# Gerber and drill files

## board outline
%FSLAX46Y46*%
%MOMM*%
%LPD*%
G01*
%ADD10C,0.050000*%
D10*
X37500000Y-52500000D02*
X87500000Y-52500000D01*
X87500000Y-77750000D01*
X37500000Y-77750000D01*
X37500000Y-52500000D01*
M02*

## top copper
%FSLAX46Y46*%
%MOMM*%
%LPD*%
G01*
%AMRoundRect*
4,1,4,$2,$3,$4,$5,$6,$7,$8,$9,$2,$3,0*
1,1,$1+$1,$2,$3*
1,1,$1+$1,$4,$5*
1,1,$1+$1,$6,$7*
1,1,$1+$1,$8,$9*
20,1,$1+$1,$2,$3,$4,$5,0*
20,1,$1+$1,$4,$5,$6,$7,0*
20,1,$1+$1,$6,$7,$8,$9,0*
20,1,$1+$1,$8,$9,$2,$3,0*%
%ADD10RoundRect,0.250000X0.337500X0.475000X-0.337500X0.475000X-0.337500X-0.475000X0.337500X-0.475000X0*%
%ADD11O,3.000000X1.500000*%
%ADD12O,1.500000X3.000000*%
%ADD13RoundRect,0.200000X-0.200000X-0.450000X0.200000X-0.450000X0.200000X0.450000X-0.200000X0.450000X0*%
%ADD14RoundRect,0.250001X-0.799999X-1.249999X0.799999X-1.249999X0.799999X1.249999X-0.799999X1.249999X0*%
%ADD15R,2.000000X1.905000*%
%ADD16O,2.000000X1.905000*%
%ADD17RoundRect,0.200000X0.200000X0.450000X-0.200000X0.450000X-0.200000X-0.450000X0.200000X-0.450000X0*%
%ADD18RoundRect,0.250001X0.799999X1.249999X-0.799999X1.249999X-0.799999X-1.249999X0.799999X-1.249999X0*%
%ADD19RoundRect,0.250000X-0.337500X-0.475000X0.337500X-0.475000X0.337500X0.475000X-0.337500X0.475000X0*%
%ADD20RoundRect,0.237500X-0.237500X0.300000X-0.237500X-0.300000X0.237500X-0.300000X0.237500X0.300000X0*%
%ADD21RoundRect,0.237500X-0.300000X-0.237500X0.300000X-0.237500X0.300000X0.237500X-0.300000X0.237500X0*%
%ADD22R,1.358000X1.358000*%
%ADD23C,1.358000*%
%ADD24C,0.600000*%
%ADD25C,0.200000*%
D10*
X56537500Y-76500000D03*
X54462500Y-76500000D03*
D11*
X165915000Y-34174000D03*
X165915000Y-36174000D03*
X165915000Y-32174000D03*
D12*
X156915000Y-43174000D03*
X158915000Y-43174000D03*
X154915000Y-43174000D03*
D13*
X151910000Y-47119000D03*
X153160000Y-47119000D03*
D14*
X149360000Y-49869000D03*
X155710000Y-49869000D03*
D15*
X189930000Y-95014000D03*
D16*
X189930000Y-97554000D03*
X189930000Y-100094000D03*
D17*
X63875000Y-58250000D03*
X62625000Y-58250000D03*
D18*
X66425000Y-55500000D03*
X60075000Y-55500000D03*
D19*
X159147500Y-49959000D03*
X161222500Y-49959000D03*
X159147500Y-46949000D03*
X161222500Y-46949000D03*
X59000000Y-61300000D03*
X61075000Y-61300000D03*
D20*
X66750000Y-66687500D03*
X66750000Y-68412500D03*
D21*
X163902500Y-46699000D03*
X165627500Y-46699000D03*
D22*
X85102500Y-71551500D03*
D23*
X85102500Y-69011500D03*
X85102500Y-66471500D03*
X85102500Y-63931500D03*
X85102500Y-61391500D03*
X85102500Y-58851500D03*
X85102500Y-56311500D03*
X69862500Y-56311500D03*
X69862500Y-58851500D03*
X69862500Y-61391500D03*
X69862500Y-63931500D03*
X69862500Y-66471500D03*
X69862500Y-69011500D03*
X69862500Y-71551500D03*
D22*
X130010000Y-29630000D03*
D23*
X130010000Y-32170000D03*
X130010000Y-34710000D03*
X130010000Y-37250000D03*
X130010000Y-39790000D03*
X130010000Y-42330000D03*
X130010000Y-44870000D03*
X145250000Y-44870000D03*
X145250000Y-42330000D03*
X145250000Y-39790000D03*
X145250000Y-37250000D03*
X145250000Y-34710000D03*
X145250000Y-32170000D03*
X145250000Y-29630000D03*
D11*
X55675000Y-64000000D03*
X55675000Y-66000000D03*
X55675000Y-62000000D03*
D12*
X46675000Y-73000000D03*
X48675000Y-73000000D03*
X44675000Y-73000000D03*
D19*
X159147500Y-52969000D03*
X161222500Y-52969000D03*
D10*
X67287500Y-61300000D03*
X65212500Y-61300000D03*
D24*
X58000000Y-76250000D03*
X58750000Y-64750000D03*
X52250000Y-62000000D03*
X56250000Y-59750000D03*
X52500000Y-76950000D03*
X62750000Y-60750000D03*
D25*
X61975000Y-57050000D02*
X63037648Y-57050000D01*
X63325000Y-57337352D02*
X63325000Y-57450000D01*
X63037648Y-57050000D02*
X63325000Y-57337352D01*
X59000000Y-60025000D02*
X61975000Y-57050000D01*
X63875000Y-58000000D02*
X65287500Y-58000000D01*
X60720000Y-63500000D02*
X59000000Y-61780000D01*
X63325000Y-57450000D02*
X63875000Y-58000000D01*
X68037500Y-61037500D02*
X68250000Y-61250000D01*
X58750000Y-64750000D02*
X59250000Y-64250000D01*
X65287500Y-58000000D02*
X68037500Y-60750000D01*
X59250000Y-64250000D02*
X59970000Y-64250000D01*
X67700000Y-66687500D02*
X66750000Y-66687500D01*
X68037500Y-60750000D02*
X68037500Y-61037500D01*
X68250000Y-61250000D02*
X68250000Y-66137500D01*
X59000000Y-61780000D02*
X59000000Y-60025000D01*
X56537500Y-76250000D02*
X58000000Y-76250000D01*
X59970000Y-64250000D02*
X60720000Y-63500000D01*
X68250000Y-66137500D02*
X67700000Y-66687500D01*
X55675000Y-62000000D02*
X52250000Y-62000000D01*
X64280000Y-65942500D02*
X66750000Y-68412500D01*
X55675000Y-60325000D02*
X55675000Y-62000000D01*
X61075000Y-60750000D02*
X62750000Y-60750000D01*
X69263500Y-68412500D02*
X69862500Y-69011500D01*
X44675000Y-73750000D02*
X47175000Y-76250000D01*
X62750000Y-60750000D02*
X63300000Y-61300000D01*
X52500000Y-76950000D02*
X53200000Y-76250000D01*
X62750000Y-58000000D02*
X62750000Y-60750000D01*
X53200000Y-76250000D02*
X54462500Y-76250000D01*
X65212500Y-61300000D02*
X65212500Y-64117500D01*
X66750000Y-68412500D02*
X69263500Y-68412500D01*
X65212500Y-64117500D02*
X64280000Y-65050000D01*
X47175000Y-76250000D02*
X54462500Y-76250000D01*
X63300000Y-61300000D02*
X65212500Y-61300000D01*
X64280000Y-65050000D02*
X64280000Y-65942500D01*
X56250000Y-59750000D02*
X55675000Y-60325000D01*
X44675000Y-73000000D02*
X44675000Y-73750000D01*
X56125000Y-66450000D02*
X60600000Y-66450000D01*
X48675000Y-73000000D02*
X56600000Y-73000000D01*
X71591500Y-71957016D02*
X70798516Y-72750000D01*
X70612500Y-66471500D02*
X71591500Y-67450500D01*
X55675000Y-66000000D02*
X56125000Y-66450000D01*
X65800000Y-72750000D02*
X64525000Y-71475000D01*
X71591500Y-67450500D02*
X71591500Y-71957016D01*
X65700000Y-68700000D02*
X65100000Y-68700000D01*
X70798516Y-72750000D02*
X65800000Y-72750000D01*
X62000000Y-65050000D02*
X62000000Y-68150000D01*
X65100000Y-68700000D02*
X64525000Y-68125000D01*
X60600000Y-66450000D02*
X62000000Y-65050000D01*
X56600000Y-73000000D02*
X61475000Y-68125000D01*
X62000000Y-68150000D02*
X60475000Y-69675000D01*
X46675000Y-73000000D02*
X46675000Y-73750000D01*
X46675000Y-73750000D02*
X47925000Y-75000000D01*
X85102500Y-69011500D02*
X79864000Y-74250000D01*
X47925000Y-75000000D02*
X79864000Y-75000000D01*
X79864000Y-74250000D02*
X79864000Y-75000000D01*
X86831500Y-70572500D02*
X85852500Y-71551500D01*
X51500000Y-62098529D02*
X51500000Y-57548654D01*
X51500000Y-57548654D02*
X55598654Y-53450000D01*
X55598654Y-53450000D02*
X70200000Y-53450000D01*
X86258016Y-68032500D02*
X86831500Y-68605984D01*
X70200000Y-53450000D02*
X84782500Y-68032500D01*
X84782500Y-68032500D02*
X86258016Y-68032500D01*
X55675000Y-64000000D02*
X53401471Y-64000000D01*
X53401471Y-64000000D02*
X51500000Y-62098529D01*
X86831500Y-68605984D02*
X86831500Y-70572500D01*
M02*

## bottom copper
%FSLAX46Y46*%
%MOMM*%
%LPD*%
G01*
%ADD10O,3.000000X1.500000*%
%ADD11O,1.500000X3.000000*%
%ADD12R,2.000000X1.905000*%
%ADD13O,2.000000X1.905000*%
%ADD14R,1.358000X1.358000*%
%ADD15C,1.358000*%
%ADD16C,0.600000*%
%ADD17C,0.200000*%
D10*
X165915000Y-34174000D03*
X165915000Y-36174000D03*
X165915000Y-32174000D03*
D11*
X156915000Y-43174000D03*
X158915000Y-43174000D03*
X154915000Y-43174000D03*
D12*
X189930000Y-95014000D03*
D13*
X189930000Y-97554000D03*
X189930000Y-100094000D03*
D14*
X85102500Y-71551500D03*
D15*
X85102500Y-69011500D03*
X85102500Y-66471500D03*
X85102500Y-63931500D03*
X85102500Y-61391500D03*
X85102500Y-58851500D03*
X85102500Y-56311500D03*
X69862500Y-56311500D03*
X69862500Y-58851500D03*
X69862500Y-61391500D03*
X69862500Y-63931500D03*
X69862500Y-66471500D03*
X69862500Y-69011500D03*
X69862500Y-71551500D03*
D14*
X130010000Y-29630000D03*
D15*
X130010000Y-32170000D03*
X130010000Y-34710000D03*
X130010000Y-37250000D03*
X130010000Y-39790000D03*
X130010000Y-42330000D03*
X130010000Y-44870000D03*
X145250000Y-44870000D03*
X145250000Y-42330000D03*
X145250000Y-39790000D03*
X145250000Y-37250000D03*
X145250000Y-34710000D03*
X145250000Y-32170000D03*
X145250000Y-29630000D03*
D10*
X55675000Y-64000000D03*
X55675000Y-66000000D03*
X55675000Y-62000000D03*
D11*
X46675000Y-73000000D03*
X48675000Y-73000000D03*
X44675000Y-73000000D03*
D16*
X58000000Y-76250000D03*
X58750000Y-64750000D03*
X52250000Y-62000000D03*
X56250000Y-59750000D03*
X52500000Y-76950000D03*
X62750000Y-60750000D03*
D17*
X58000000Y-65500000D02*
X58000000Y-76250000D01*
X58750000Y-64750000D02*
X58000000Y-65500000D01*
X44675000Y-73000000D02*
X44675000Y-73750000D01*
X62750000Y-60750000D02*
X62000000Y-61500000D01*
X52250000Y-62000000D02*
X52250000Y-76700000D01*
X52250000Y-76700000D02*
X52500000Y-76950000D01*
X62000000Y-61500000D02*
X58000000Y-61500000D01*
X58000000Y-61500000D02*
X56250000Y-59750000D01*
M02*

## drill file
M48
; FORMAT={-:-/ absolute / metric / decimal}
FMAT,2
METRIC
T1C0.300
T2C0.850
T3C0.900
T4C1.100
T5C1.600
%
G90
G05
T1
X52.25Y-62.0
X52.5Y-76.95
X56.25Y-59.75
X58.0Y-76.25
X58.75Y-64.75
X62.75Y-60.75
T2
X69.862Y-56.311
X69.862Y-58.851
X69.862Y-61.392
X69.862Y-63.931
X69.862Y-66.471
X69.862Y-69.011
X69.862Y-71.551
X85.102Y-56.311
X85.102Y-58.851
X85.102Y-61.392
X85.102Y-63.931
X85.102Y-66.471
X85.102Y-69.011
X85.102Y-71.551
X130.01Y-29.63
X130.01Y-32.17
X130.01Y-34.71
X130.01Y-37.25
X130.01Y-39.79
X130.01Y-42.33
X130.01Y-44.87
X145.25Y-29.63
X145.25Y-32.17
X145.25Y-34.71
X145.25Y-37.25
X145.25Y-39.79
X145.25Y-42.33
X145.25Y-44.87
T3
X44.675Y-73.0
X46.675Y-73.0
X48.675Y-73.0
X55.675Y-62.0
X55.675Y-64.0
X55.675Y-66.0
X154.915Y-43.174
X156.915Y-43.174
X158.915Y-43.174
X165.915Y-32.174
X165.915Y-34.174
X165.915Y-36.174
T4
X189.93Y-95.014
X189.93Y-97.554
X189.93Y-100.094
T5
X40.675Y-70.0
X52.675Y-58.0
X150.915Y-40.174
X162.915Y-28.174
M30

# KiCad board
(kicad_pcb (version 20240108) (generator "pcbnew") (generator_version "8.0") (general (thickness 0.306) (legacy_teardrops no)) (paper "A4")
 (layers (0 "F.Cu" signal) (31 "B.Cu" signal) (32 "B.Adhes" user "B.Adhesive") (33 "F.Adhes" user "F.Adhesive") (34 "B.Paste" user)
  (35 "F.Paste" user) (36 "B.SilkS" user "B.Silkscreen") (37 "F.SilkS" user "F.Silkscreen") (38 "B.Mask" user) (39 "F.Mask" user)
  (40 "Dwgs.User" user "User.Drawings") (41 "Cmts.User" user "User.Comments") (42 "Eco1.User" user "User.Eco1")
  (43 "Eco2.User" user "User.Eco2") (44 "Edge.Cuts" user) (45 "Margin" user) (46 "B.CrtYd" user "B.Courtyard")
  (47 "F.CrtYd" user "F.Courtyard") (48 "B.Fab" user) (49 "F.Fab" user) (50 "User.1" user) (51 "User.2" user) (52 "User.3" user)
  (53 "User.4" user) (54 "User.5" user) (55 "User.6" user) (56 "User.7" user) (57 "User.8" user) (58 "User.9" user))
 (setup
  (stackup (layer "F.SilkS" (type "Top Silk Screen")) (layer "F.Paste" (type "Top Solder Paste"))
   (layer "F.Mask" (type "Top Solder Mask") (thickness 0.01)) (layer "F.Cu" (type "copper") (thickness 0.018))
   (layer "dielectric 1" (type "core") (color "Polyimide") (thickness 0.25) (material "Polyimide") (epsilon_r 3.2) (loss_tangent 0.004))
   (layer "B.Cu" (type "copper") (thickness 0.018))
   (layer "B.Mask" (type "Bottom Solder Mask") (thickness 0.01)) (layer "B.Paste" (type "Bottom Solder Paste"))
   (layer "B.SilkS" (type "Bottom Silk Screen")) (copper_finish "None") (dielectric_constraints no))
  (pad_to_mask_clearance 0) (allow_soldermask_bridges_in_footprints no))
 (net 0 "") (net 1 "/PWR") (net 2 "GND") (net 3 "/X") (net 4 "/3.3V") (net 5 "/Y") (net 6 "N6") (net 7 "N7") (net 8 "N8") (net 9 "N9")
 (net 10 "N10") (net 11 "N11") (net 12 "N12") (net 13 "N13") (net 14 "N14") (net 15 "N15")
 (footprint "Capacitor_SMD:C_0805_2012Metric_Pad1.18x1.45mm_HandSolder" (layer "F.Cu") (at 55.5 76.5 180)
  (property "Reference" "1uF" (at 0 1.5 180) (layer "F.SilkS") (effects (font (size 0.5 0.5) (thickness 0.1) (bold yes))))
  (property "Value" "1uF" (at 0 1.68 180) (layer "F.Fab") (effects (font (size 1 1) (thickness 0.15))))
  (pad "1" smd roundrect (at -1.0375 0 180) (size 1.175 1.45) (layers "F.Cu" "F.Paste" "F.Mask") (roundrect_rratio 0.212766) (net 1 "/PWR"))
  (pad "2" smd roundrect (at 1.0375 0 180) (size 1.175 1.45) (layers "F.Cu" "F.Paste" "F.Mask") (roundrect_rratio 0.212766) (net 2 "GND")))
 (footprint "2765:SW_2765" (layer "F.Cu") (at 156.915 34.174)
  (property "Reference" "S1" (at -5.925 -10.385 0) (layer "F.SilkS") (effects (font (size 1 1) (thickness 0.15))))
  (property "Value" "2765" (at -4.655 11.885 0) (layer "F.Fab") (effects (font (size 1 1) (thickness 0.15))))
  (pad "" np_thru_hole circle (at -6 6) (size 1.6 1.6) (drill 1.6) (layers "*.Cu" "*.Mask"))
  (pad "" np_thru_hole circle (at 6 -6) (size 1.6 1.6) (drill 1.6) (layers "*.Cu" "*.Mask"))
  (pad "X" thru_hole oval (at 9 0) (size 3 1.5) (drill 0.9) (layers "*.Cu" "*.Mask") (remove_unused_layers no) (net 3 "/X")
   (solder_mask_margin 0.102))
  (pad "X+" thru_hole oval (at 9 2) (size 3 1.5) (drill 0.9) (layers "*.Cu" "*.Mask") (remove_unused_layers no) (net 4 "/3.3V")
   (solder_mask_margin 0.102))
  (pad "X-" thru_hole oval (at 9 -2) (size 3 1.5) (drill 0.9) (layers "*.Cu" "*.Mask") (remove_unused_layers no) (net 2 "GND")
   (solder_mask_margin 0.102))
  (pad "Y" thru_hole oval (at 0 9) (size 1.5 3) (drill 0.9) (layers "*.Cu" "*.Mask") (remove_unused_layers no) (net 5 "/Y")
   (solder_mask_margin 0.102))
  (pad "Y+" thru_hole oval (at 2 9) (size 1.5 3) (drill 0.9) (layers "*.Cu" "*.Mask") (remove_unused_layers no) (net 4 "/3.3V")
   (solder_mask_margin 0.102))
  (pad "Y-" thru_hole oval (at -2 9) (size 1.5 3) (drill 0.9) (layers "*.Cu" "*.Mask") (remove_unused_layers no) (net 2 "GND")
   (solder_mask_margin 0.102)))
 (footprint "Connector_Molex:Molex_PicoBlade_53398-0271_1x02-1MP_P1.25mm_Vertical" (layer "F.Cu") (at 152.535 48.369)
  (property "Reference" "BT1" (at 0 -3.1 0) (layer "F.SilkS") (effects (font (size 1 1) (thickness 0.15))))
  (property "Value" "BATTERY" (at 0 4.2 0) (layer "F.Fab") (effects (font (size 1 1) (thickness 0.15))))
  (pad "1" smd roundrect (at -0.625 -1.25) (size 0.8 1.3) (layers "F.Cu" "F.Paste" "F.Mask") (roundrect_rratio 0.25) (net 1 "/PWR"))
  (pad "2" smd roundrect (at 0.625 -1.25) (size 0.8 1.3) (layers "F.Cu" "F.Paste" "F.Mask") (roundrect_rratio 0.25) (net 2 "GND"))
  (pad "MP" smd roundrect (at -3.175 1.5) (size 2.1 3) (layers "F.Cu" "F.Paste" "F.Mask") (roundrect_rratio 0.119048))
  (pad "MP" smd roundrect (at 3.175 1.5) (size 2.1 3) (layers "F.Cu" "F.Paste" "F.Mask") (roundrect_rratio 0.119048)))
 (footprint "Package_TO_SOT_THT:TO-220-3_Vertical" (layer "F.Cu") (at 189.93 95.014 -90)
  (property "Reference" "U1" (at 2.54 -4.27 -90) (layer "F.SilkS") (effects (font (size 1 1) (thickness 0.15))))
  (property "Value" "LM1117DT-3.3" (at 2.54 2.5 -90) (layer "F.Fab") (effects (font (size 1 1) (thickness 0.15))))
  (pad "1" thru_hole rect (at 0 0 270) (size 1.905 2) (drill 1.1) (layers "*.Cu" "*.Mask") (remove_unused_layers no) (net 2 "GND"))
  (pad "2" thru_hole oval (at 2.54 0 270) (size 1.905 2) (drill 1.1) (layers "*.Cu" "*.Mask") (remove_unused_layers no) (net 4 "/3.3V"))
  (pad "3" thru_hole oval (at 5.08 0 270) (size 1.905 2) (drill 1.1) (layers "*.Cu" "*.Mask") (remove_unused_layers no) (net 1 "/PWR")))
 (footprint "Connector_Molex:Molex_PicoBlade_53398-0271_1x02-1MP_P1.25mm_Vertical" (layer "F.Cu") (at 63.25 57 180)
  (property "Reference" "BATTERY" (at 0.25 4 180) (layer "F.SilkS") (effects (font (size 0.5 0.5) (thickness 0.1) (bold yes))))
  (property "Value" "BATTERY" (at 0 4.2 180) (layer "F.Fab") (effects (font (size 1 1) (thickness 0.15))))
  (pad "1" smd roundrect (at -0.625 -1.25 180) (size 0.8 1.3) (layers "F.Cu" "F.Paste" "F.Mask") (roundrect_rratio 0.25) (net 1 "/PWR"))
  (pad "2" smd roundrect (at 0.625 -1.25 180) (size 0.8 1.3) (layers "F.Cu" "F.Paste" "F.Mask") (roundrect_rratio 0.25) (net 2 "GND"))
  (pad "MP" smd roundrect (at -3.175 1.5 180) (size 2.1 3) (layers "F.Cu" "F.Paste" "F.Mask") (roundrect_rratio 0.119048))
  (pad "MP" smd roundrect (at 3.175 1.5 180) (size 2.1 3) (layers "F.Cu" "F.Paste" "F.Mask") (roundrect_rratio 0.119048)))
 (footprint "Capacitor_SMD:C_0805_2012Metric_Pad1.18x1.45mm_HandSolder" (layer "F.Cu") (at 160.185 49.959)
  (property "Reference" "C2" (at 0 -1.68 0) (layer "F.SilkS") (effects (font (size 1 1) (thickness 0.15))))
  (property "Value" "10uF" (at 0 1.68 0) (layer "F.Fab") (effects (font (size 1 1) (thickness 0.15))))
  (pad "1" smd roundrect (at -1.0375 0) (size 1.175 1.45) (layers "F.Cu" "F.Paste" "F.Mask") (roundrect_rratio 0.212766) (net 1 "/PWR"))
  (pad "2" smd roundrect (at 1.0375 0) (size 1.175 1.45) (layers "F.Cu" "F.Paste" "F.Mask") (roundrect_rratio 0.212766) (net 2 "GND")))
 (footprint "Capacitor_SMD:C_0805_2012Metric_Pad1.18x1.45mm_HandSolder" (layer "F.Cu") (at 160.185 46.949)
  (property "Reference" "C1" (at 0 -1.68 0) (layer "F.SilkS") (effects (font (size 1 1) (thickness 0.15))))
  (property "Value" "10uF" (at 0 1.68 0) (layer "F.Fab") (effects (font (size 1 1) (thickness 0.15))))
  (pad "1" smd roundrect (at -1.0375 0) (size 1.175 1.45) (layers "F.Cu" "F.Paste" "F.Mask") (roundrect_rratio 0.212766) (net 1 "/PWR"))
  (pad "2" smd roundrect (at 1.0375 0) (size 1.175 1.45) (layers "F.Cu" "F.Paste" "F.Mask") (roundrect_rratio 0.212766) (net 2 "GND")))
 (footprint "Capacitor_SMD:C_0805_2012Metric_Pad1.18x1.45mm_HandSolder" (layer "F.Cu") (at 60.0375 61.3)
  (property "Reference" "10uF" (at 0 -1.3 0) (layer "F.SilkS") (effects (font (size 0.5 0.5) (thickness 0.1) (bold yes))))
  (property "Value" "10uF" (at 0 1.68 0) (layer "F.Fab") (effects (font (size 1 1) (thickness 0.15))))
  (pad "1" smd roundrect (at -1.0375 0) (size 1.175 1.45) (layers "F.Cu" "F.Paste" "F.Mask") (roundrect_rratio 0.212766) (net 1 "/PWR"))
  (pad "2" smd roundrect (at 1.0375 0) (size 1.175 1.45) (layers "F.Cu" "F.Paste" "F.Mask") (roundrect_rratio 0.212766) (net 2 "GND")))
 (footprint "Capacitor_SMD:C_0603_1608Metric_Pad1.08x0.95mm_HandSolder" (layer "F.Cu") (at 66.75 67.55 -90)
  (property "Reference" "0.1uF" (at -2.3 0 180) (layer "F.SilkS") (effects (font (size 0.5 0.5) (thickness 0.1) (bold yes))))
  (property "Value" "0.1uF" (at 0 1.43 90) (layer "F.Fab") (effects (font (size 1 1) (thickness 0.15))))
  (pad "1" smd roundrect (at -0.8625 0 270) (size 1.075 0.95) (layers "F.Cu" "F.Paste" "F.Mask") (roundrect_rratio 0.25) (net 1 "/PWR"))
  (pad "2" smd roundrect (at 0.8625 0 270) (size 1.075 0.95) (layers "F.Cu" "F.Paste" "F.Mask") (roundrect_rratio 0.25) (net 2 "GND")))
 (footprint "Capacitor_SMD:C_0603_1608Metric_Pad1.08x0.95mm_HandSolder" (layer "F.Cu") (at 164.765 46.699)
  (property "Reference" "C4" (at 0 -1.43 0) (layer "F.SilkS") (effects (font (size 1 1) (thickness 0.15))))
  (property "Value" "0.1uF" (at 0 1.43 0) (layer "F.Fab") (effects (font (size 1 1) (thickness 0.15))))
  (pad "1" smd roundrect (at -0.8625 0) (size 1.075 0.95) (layers "F.Cu" "F.Paste" "F.Mask") (roundrect_rratio 0.25) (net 1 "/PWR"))
  (pad "2" smd roundrect (at 0.8625 0) (size 1.075 0.95) (layers "F.Cu" "F.Paste" "F.Mask") (roundrect_rratio 0.25) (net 2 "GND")))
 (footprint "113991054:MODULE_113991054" (layer "F.Cu") (at 77.4825 63.995 180)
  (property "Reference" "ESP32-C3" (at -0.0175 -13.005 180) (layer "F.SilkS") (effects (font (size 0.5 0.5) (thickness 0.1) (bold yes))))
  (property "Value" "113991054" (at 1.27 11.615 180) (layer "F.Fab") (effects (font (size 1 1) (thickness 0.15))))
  (pad "1" thru_hole rect (at -7.62 -7.5565 180) (size 1.358 1.358) (drill 0.85) (layers "*.Cu" "*.Mask") (remove_unused_layers no)
   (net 3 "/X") (solder_mask_margin 0.102))
  (pad "2" thru_hole circle (at -7.62 -5.0165 180) (size 1.358 1.358) (drill 0.85) (layers "*.Cu" "*.Mask") (remove_unused_layers no)
   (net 5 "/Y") (solder_mask_margin 0.102))
  (pad "3" thru_hole circle (at -7.62 -2.4765 180) (size 1.358 1.358) (drill 0.85) (layers "*.Cu" "*.Mask") (remove_unused_layers no)
   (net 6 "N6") (solder_mask_margin 0.102))
  (pad "4" thru_hole circle (at -7.62 0.0635 180) (size 1.358 1.358) (drill 0.85) (layers "*.Cu" "*.Mask") (remove_unused_layers no)
   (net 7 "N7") (solder_mask_margin 0.102))
  (pad "5" thru_hole circle (at -7.62 2.6035 180) (size 1.358 1.358) (drill 0.85) (layers "*.Cu" "*.Mask") (remove_unused_layers no)
   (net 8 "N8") (solder_mask_margin 0.102))
  (pad "6" thru_hole circle (at -7.62 5.1435 180) (size 1.358 1.358) (drill 0.85) (layers "*.Cu" "*.Mask") (remove_unused_layers no)
   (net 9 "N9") (solder_mask_margin 0.102))
  (pad "7" thru_hole circle (at -7.62 7.6835 180) (size 1.358 1.358) (drill 0.85) (layers "*.Cu" "*.Mask") (remove_unused_layers no)
   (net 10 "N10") (solder_mask_margin 0.102))
  (pad "8" thru_hole circle (at 7.62 7.6835 180) (size 1.358 1.358) (drill 0.85) (layers "*.Cu" "*.Mask") (remove_unused_layers no)
   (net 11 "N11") (solder_mask_margin 0.102))
  (pad "9" thru_hole circle (at 7.62 5.1435 180) (size 1.358 1.358) (drill 0.85) (layers "*.Cu" "*.Mask") (remove_unused_layers no)
   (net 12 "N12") (solder_mask_margin 0.102))
  (pad "10" thru_hole circle (at 7.62 2.6035 180) (size 1.358 1.358) (drill 0.85) (layers "*.Cu" "*.Mask") (remove_unused_layers no)
   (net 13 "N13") (solder_mask_margin 0.102))
  (pad "11" thru_hole circle (at 7.62 0.0635 180) (size 1.358 1.358) (drill 0.85) (layers "*.Cu" "*.Mask") (remove_unused_layers no)
   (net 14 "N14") (solder_mask_margin 0.102))
  (pad "12" thru_hole circle (at 7.62 -2.4765 180) (size 1.358 1.358) (drill 0.85) (layers "*.Cu" "*.Mask") (remove_unused_layers no)
   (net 4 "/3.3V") (solder_mask_margin 0.102))
  (pad "13" thru_hole circle (at 7.62 -5.0165 180) (size 1.358 1.358) (drill 0.85) (layers "*.Cu" "*.Mask") (remove_unused_layers no)
   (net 2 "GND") (solder_mask_margin 0.102))
  (pad "14" thru_hole circle (at 7.62 -7.5565 180) (size 1.358 1.358) (drill 0.85) (layers "*.Cu" "*.Mask") (remove_unused_layers no)
   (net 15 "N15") (solder_mask_margin 0.102)))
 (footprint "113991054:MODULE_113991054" (layer "F.Cu") (at 137.63 37.1865)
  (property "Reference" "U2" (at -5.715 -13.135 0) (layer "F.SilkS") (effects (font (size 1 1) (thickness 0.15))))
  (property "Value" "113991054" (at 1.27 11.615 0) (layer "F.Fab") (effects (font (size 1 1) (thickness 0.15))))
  (pad "1" thru_hole rect (at -7.62 -7.5565) (size 1.358 1.358) (drill 0.85) (layers "*.Cu" "*.Mask") (remove_unused_layers no) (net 3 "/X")
   (solder_mask_margin 0.102))
  (pad "2" thru_hole circle (at -7.62 -5.0165) (size 1.358 1.358) (drill 0.85) (layers "*.Cu" "*.Mask") (remove_unused_layers no)
   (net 5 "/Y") (solder_mask_margin 0.102))
  (pad "3" thru_hole circle (at -7.62 -2.4765) (size 1.358 1.358) (drill 0.85) (layers "*.Cu" "*.Mask") (remove_unused_layers no)
   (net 6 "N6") (solder_mask_margin 0.102))
  (pad "4" thru_hole circle (at -7.62 0.0635) (size 1.358 1.358) (drill 0.85) (layers "*.Cu" "*.Mask") (remove_unused_layers no)
   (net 7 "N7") (solder_mask_margin 0.102))
  (pad "5" thru_hole circle (at -7.62 2.6035) (size 1.358 1.358) (drill 0.85) (layers "*.Cu" "*.Mask") (remove_unused_layers no)
   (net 8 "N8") (solder_mask_margin 0.102))
  (pad "6" thru_hole circle (at -7.62 5.1435) (size 1.358 1.358) (drill 0.85) (layers "*.Cu" "*.Mask") (remove_unused_layers no)
   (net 9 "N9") (solder_mask_margin 0.102))
  (pad "7" thru_hole circle (at -7.62 7.6835) (size 1.358 1.358) (drill 0.85) (layers "*.Cu" "*.Mask") (remove_unused_layers no)
   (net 10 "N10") (solder_mask_margin 0.102))
  (pad "8" thru_hole circle (at 7.62 7.6835) (size 1.358 1.358) (drill 0.85) (layers "*.Cu" "*.Mask") (remove_unused_layers no)
   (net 11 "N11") (solder_mask_margin 0.102))
  (pad "9" thru_hole circle (at 7.62 5.1435) (size 1.358 1.358) (drill 0.85) (layers "*.Cu" "*.Mask") (remove_unused_layers no)
   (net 12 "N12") (solder_mask_margin 0.102))
  (pad "10" thru_hole circle (at 7.62 2.6035) (size 1.358 1.358) (drill 0.85) (layers "*.Cu" "*.Mask") (remove_unused_layers no)
   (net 13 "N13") (solder_mask_margin 0.102))
  (pad "11" thru_hole circle (at 7.62 0.0635) (size 1.358 1.358) (drill 0.85) (layers "*.Cu" "*.Mask") (remove_unused_layers no)
   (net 14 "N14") (solder_mask_margin 0.102))
  (pad "12" thru_hole circle (at 7.62 -2.4765) (size 1.358 1.358) (drill 0.85) (layers "*.Cu" "*.Mask") (remove_unused_layers no)
   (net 4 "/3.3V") (solder_mask_margin 0.102))
  (pad "13" thru_hole circle (at 7.62 -5.0165) (size 1.358 1.358) (drill 0.85) (layers "*.Cu" "*.Mask") (remove_unused_layers no)
   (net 2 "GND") (solder_mask_margin 0.102))
  (pad "14" thru_hole circle (at 7.62 -7.5565) (size 1.358 1.358) (drill 0.85) (layers "*.Cu" "*.Mask") (remove_unused_layers no)
   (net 15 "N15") (solder_mask_margin 0.102)))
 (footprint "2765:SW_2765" (layer "F.Cu") (at 46.675 64)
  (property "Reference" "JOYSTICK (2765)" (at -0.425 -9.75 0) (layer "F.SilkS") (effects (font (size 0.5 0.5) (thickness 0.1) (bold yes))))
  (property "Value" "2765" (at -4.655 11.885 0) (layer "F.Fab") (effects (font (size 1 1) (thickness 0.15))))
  (pad "" np_thru_hole circle (at -6 6) (size 1.6 1.6) (drill 1.6) (layers "*.Cu" "*.Mask"))
  (pad "" np_thru_hole circle (at 6 -6) (size 1.6 1.6) (drill 1.6) (layers "*.Cu" "*.Mask"))
  (pad "X" thru_hole oval (at 9 0) (size 3 1.5) (drill 0.9) (layers "*.Cu" "*.Mask") (remove_unused_layers no) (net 3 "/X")
   (solder_mask_margin 0.102))
  (pad "X+" thru_hole oval (at 9 2) (size 3 1.5) (drill 0.9) (layers "*.Cu" "*.Mask") (remove_unused_layers no) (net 4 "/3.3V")
   (solder_mask_margin 0.102))
  (pad "X-" thru_hole oval (at 9 -2) (size 3 1.5) (drill 0.9) (layers "*.Cu" "*.Mask") (remove_unused_layers no) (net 2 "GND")
   (solder_mask_margin 0.102))
  (pad "Y" thru_hole oval (at 0 9) (size 1.5 3) (drill 0.9) (layers "*.Cu" "*.Mask") (remove_unused_layers no) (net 5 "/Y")
   (solder_mask_margin 0.102))
  (pad "Y+" thru_hole oval (at 2 9) (size 1.5 3) (drill 0.9) (layers "*.Cu" "*.Mask") (remove_unused_layers no) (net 4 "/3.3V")
   (solder_mask_margin 0.102))
  (pad "Y-" thru_hole oval (at -2 9) (size 1.5 3) (drill 0.9) (layers "*.Cu" "*.Mask") (remove_unused_layers no) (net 2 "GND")
   (solder_mask_margin 0.102)))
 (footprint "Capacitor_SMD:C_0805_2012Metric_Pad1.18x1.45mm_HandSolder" (layer "F.Cu") (at 160.185 52.969)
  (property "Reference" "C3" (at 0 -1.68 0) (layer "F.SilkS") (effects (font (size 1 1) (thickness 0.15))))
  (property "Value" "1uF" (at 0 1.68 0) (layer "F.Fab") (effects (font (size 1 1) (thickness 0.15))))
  (pad "1" smd roundrect (at -1.0375 0) (size 1.175 1.45) (layers "F.Cu" "F.Paste" "F.Mask") (roundrect_rratio 0.212766) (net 1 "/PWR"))
  (pad "2" smd roundrect (at 1.0375 0) (size 1.175 1.45) (layers "F.Cu" "F.Paste" "F.Mask") (roundrect_rratio 0.212766) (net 2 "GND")))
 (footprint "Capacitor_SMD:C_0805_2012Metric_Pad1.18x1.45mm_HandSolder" (layer "F.Cu") (at 66.25 61.3 180)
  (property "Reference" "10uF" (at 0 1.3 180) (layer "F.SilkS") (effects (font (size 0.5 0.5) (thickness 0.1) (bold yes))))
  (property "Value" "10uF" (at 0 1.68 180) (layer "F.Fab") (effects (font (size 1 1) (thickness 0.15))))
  (pad "1" smd roundrect (at -1.0375 0 180) (size 1.175 1.45) (layers "F.Cu" "F.Paste" "F.Mask") (roundrect_rratio 0.212766) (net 1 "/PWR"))
  (pad "2" smd roundrect (at 1.0375 0 180) (size 1.175 1.45) (layers "F.Cu" "F.Paste" "F.Mask") (roundrect_rratio 0.212766) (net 2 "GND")))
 (gr_rect (start 37.5 52.5) (end 87.5 77.75) (stroke (width 0.05) (type default)) (fill none) (layer "Edge.Cuts"))
 (segment (start 61.975 57.05) (end 63.037648 57.05) (width 0.2) (layer "F.Cu") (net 1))
 (segment (start 63.325 57.337352) (end 63.325 57.45) (width 0.2) (layer "F.Cu") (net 1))
 (segment (start 63.037648 57.05) (end 63.325 57.337352) (width 0.2) (layer "F.Cu") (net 1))
 (segment (start 59 60.025) (end 61.975 57.05) (width 0.2) (layer "F.Cu") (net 1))
 (segment (start 63.875 58) (end 65.2875 58) (width 0.2) (layer "F.Cu") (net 1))
 (segment (start 60.72 63.5) (end 59 61.78) (width 0.2) (layer "F.Cu") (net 1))
 (segment (start 63.325 57.45) (end 63.875 58) (width 0.2) (layer "F.Cu") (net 1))
 (segment (start 68.0375 61.0375) (end 68.25 61.25) (width 0.2) (layer "F.Cu") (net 1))
 (segment (start 58.75 64.75) (end 59.25 64.25) (width 0.2) (layer "F.Cu") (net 1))
 (segment (start 65.2875 58) (end 68.0375 60.75) (width 0.2) (layer "F.Cu") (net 1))
 (segment (start 59.25 64.25) (end 59.97 64.25) (width 0.2) (layer "F.Cu") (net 1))
 (segment (start 67.7 66.6875) (end 66.75 66.6875) (width 0.2) (layer "F.Cu") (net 1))
 (segment (start 68.0375 60.75) (end 68.0375 61.0375) (width 0.2) (layer "F.Cu") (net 1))
 (segment (start 68.25 61.25) (end 68.25 66.1375) (width 0.2) (layer "F.Cu") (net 1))
 (segment (start 59 61.78) (end 59 60.025) (width 0.2) (layer "F.Cu") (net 1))
 (segment (start 56.5375 76.25) (end 58 76.25) (width 0.2) (layer "F.Cu") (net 1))
 (segment (start 59.97 64.25) (end 60.72 63.5) (width 0.2) (layer "F.Cu") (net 1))
 (segment (start 68.25 66.1375) (end 67.7 66.6875) (width 0.2) (layer "F.Cu") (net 1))
 (via (at 58 76.25) (size 0.6) (drill 0.3) (layers "F.Cu" "B.Cu") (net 1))
 (via (at 58.75 64.75) (size 0.6) (drill 0.3) (layers "F.Cu" "B.Cu") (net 1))
 (segment (start 58 65.5) (end 58 76.25) (width 0.2) (layer "B.Cu") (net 1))
 (segment (start 58.75 64.75) (end 58 65.5) (width 0.2) (layer "B.Cu") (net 1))
 (segment (start 55.675 62) (end 52.25 62) (width 0.2) (layer "F.Cu") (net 2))
 (segment (start 64.28 65.9425) (end 66.75 68.4125) (width 0.2) (layer "F.Cu") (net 2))
 (segment (start 55.675 60.325) (end 55.675 62) (width 0.2) (layer "F.Cu") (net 2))
 (segment (start 61.075 60.75) (end 62.75 60.75) (width 0.2) (layer "F.Cu") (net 2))
 (segment (start 69.2635 68.4125) (end 69.8625 69.0115) (width 0.2) (layer "F.Cu") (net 2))
 (segment (start 44.675 73.75) (end 47.175 76.25) (width 0.2) (layer "F.Cu") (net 2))
 (segment (start 62.75 60.75) (end 63.3 61.3) (width 0.2) (layer "F.Cu") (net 2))
 (segment (start 52.5 76.95) (end 53.2 76.25) (width 0.2) (layer "F.Cu") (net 2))
 (segment (start 62.75 58) (end 62.75 60.75) (width 0.2) (layer "F.Cu") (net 2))
 (segment (start 53.2 76.25) (end 54.4625 76.25) (width 0.2) (layer "F.Cu") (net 2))
 (segment (start 65.2125 61.3) (end 65.2125 64.1175) (width 0.2) (layer "F.Cu") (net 2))
 (segment (start 66.75 68.4125) (end 69.2635 68.4125) (width 0.2) (layer "F.Cu") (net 2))
 (segment (start 65.2125 64.1175) (end 64.28 65.05) (width 0.2) (layer "F.Cu") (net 2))
 (segment (start 47.175 76.25) (end 54.4625 76.25) (width 0.2) (layer "F.Cu") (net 2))
 (segment (start 63.3 61.3) (end 65.2125 61.3) (width 0.2) (layer "F.Cu") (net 2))
 (segment (start 64.28 65.05) (end 64.28 65.9425) (width 0.2) (layer "F.Cu") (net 2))
 (segment (start 56.25 59.75) (end 55.675 60.325) (width 0.2) (layer "F.Cu") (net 2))
 (segment (start 44.675 73) (end 44.675 73.75) (width 0.2) (layer "F.Cu") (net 2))
 (via (at 52.25 62) (size 0.6) (drill 0.3) (layers "F.Cu" "B.Cu") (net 2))
 (via (at 56.25 59.75) (size 0.6) (drill 0.3) (layers "F.Cu" "B.Cu") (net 2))
 (via (at 52.5 76.95) (size 0.6) (drill 0.3) (layers "F.Cu" "B.Cu") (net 2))
 (via (at 62.75 60.75) (size 0.6) (drill 0.3) (layers "F.Cu" "B.Cu") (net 2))
 (segment (start 44.675 73) (end 44.675 73.75) (width 0.2) (layer "B.Cu") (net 2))
 (segment (start 62.75 60.75) (end 62 61.5) (width 0.2) (layer "B.Cu") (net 2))
 (segment (start 52.25 62) (end 52.25 76.7) (width 0.2) (layer "B.Cu") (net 2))
 (segment (start 52.25 76.7) (end 52.5 76.95) (width 0.2) (layer "B.Cu") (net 2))
 (segment (start 62 61.5) (end 58 61.5) (width 0.2) (layer "B.Cu") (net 2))
 (segment (start 58 61.5) (end 56.25 59.75) (width 0.2) (layer "B.Cu") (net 2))
 (segment (start 56.125 66.45) (end 60.6 66.45) (width 0.2) (layer "F.Cu") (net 4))
 (segment (start 48.675 73) (end 56.6 73) (width 0.2) (layer "F.Cu") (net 4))
 (segment (start 71.5915 71.957016) (end 70.798516 72.75) (width 0.2) (layer "F.Cu") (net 4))
 (segment (start 70.6125 66.4715) (end 71.5915 67.4505) (width 0.2) (layer "F.Cu") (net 4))
 (segment (start 55.675 66) (end 56.125 66.45) (width 0.2) (layer "F.Cu") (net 4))
 (segment (start 65.8 72.75) (end 64.525 71.475) (width 0.2) (layer "F.Cu") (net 4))
 (segment (start 71.5915 67.4505) (end 71.5915 71.957016) (width 0.2) (layer "F.Cu") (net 4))
 (segment (start 65.7 68.7) (end 65.1 68.7) (width 0.2) (layer "F.Cu") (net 4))
 (segment (start 70.798516 72.75) (end 65.8 72.75) (width 0.2) (layer "F.Cu") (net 4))
 (segment (start 62 65.05) (end 62 68.15) (width 0.2) (layer "F.Cu") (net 4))
 (segment (start 65.1 68.7) (end 64.525 68.125) (width 0.2) (layer "F.Cu") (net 4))
 (segment (start 60.6 66.45) (end 62 65.05) (width 0.2) (layer "F.Cu") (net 4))
 (segment (start 56.6 73) (end 61.475 68.125) (width 0.2) (layer "F.Cu") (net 4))
 (segment (start 62 68.15) (end 60.475 69.675) (width 0.2) (layer "F.Cu") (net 4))
 (segment (start 46.675 73) (end 46.675 73.75) (width 0.2) (layer "F.Cu") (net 5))
 (segment (start 46.675 73.75) (end 47.925 75) (width 0.2) (layer "F.Cu") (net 5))
 (segment (start 85.1025 69.0115) (end 79.864 74.25) (width 0.2) (layer "F.Cu") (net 5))
 (segment (start 47.925 75) (end 79.864 75) (width 0.2) (layer "F.Cu") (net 5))
 (segment (start 79.864 74.25) (end 79.864 75) (width 0.2) (layer "F.Cu") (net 5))
 (segment (start 86.8315 70.5725) (end 85.8525 71.5515) (width 0.2) (layer "F.Cu") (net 3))
 (segment (start 51.5 62.098529) (end 51.5 57.548654) (width 0.2) (layer "F.Cu") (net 3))
 (segment (start 51.5 57.548654) (end 55.598654 53.45) (width 0.2) (layer "F.Cu") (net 3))
 (segment (start 55.598654 53.45) (end 70.2 53.45) (width 0.2) (layer "F.Cu") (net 3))
 (segment (start 86.258016 68.0325) (end 86.8315 68.605984) (width 0.2) (layer "F.Cu") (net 3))
 (segment (start 70.2 53.45) (end 84.7825 68.0325) (width 0.2) (layer "F.Cu") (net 3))
 (segment (start 84.7825 68.0325) (end 86.258016 68.0325) (width 0.2) (layer "F.Cu") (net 3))
 (segment (start 55.675 64) (end 53.401471 64) (width 0.2) (layer "F.Cu") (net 3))
 (segment (start 53.401471 64) (end 51.5 62.098529) (width 0.2) (layer "F.Cu") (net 3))
 (segment (start 86.8315 68.605984) (end 86.8315 70.5725) (width 0.2) (layer "F.Cu") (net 3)))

